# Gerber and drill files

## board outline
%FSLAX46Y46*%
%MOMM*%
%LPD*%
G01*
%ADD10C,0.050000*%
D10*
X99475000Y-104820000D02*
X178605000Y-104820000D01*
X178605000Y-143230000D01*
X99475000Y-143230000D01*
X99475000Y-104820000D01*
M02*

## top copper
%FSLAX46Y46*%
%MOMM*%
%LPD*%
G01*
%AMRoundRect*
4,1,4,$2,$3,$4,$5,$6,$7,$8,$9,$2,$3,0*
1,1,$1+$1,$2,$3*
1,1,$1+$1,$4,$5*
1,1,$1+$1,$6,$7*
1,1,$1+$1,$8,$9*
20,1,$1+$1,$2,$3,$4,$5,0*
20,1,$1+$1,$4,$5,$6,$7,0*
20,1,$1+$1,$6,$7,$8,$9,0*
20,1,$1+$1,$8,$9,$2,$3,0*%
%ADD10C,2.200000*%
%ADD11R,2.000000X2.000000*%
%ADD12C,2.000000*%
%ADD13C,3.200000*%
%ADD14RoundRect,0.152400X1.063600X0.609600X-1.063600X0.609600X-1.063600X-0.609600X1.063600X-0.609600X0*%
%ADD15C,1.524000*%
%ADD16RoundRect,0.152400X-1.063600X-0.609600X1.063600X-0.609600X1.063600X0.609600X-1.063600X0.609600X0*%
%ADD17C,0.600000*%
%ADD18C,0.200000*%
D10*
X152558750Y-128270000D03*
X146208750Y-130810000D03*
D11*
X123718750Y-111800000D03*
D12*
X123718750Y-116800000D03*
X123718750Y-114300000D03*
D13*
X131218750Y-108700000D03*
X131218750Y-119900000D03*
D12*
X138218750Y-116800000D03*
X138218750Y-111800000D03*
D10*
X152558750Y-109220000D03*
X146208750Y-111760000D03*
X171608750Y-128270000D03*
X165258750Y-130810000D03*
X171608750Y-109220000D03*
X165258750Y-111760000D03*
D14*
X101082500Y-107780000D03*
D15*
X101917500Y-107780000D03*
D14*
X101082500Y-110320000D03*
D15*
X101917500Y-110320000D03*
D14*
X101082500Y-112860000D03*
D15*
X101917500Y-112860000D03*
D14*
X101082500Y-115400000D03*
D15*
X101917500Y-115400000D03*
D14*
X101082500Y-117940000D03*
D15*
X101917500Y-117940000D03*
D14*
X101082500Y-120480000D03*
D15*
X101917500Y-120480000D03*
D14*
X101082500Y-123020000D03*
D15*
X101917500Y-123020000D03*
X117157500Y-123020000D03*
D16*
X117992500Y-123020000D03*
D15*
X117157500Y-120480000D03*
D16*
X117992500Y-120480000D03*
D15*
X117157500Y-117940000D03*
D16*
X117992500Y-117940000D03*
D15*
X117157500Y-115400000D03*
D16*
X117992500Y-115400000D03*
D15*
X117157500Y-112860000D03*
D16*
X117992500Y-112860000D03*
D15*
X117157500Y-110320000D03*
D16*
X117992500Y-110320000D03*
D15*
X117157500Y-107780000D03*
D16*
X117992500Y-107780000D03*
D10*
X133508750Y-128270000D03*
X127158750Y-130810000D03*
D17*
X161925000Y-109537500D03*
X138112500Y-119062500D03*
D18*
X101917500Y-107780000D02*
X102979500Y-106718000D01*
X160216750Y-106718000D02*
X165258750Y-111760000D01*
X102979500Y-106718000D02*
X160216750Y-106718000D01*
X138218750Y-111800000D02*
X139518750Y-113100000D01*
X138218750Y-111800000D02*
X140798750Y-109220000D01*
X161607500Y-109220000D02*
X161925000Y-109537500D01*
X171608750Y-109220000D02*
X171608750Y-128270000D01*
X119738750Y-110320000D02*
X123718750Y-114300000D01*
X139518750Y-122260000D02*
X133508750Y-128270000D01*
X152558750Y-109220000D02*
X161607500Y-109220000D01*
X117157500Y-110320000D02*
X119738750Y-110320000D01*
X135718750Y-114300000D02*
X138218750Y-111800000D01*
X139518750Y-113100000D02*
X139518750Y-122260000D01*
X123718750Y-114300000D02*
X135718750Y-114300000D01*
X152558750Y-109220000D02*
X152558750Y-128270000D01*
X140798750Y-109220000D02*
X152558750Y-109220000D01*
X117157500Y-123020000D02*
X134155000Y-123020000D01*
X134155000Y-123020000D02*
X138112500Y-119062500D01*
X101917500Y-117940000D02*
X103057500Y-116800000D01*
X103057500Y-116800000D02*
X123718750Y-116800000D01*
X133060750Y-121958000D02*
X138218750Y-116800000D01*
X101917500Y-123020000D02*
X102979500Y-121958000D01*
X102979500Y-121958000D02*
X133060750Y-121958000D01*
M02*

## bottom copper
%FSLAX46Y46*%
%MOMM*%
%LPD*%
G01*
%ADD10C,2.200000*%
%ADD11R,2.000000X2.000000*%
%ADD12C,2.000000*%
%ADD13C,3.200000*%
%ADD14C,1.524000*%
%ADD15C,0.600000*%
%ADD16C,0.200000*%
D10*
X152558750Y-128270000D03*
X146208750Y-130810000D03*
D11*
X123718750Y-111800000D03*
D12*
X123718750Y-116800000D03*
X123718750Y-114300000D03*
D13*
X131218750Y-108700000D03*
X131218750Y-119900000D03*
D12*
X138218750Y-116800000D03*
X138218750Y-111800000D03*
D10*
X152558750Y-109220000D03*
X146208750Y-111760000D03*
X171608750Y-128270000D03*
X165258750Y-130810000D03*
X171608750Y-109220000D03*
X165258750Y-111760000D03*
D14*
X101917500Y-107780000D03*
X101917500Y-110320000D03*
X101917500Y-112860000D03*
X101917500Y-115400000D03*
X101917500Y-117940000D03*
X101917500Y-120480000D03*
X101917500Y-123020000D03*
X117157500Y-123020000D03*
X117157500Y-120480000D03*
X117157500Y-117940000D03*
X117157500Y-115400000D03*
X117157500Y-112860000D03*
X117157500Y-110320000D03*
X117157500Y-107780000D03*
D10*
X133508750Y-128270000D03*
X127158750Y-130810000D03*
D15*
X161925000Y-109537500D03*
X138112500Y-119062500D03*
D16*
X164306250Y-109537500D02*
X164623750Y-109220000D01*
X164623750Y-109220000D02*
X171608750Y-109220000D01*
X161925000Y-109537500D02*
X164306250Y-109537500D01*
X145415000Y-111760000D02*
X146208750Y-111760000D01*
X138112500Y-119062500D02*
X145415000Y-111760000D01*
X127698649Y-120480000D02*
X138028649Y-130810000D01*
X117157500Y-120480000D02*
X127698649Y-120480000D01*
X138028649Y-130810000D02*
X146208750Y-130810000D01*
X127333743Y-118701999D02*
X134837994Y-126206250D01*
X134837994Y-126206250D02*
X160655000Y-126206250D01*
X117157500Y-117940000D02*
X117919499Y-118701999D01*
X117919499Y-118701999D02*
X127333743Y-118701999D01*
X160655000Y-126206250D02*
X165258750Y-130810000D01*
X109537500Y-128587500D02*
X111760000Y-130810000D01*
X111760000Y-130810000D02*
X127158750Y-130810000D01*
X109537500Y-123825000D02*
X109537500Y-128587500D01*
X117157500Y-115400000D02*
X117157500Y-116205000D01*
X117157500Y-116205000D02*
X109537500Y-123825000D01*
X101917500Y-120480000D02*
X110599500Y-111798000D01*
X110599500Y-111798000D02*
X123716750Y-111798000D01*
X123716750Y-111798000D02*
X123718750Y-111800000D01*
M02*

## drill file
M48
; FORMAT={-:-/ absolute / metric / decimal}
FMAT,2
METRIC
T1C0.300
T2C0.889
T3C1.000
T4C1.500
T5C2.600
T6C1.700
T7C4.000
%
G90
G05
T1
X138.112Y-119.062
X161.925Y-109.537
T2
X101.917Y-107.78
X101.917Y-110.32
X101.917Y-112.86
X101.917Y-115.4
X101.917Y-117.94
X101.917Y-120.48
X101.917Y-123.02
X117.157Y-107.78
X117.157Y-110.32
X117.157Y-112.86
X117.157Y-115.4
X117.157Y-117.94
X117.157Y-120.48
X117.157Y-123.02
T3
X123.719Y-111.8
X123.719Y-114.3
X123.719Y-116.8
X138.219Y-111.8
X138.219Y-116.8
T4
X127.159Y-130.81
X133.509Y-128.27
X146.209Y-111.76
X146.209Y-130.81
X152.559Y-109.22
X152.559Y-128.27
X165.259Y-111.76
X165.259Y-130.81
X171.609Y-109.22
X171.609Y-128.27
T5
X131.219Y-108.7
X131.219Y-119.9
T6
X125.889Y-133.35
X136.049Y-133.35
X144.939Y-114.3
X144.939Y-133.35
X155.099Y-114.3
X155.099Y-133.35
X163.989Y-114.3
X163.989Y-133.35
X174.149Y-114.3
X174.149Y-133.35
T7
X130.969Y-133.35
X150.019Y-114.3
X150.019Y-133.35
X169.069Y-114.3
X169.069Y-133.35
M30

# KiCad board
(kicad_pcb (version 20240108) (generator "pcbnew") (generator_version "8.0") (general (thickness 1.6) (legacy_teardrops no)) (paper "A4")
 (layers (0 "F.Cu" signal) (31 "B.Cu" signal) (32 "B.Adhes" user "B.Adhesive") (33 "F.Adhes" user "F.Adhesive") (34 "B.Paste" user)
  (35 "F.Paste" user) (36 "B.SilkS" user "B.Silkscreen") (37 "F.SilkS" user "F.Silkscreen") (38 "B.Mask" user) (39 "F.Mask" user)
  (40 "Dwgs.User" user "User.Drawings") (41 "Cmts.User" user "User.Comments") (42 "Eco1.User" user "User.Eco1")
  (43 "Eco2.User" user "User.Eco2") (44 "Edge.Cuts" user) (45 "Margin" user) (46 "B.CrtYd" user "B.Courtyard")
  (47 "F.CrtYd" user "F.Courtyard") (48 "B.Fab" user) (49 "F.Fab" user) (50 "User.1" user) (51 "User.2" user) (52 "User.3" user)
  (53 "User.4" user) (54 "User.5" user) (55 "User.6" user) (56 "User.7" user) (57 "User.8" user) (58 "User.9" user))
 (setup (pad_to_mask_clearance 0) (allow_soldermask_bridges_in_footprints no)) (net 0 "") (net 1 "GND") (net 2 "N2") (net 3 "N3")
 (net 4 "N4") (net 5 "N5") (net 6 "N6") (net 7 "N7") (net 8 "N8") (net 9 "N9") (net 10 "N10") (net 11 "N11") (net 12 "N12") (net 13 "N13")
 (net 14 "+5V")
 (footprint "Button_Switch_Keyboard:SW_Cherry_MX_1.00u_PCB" (layer "F.Cu") (at 152.55875 128.27)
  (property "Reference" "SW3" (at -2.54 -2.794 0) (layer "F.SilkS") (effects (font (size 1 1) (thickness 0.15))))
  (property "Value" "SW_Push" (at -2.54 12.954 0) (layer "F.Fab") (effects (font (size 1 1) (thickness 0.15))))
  (pad "" np_thru_hole circle (at -7.62 5.08) (size 1.7 1.7) (drill 1.7) (layers "*.Cu" "*.Mask"))
  (pad "" np_thru_hole circle (at -2.54 5.08) (size 4 4) (drill 4) (layers "*.Cu" "*.Mask"))
  (pad "" np_thru_hole circle (at 2.54 5.08) (size 1.7 1.7) (drill 1.7) (layers "*.Cu" "*.Mask"))
  (pad "1" thru_hole circle (at 0 0) (size 2.2 2.2) (drill 1.5) (layers "*.Cu" "*.Mask") (remove_unused_layers no) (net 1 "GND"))
  (pad "2" thru_hole circle (at -6.35 2.54) (size 2.2 2.2) (drill 1.5) (layers "*.Cu" "*.Mask") (remove_unused_layers no) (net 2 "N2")))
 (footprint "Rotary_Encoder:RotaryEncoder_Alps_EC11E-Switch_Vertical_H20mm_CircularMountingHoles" (layer "F.Cu") (at 123.71875 111.8)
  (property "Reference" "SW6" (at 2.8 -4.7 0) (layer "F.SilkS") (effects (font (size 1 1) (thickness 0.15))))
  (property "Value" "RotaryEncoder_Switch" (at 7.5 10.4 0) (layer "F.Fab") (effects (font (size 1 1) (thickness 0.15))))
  (pad "A" thru_hole rect (at 0 0) (size 2 2) (drill 1) (layers "*.Cu" "*.Mask") (remove_unused_layers no) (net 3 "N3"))
  (pad "B" thru_hole circle (at 0 5) (size 2 2) (drill 1) (layers "*.Cu" "*.Mask") (remove_unused_layers no) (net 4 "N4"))
  (pad "C" thru_hole circle (at 0 2.5) (size 2 2) (drill 1) (layers "*.Cu" "*.Mask") (remove_unused_layers no) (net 1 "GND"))
  (pad "MP" thru_hole circle (at 7.5 -3.1) (size 3.2 3.2) (drill 2.6) (layers "*.Cu" "*.Mask") (remove_unused_layers no))
  (pad "MP" thru_hole circle (at 7.5 8.1) (size 3.2 3.2) (drill 2.6) (layers "*.Cu" "*.Mask") (remove_unused_layers no))
  (pad "S1" thru_hole circle (at 14.5 5) (size 2 2) (drill 1) (layers "*.Cu" "*.Mask") (remove_unused_layers no) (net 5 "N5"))
  (pad "S2" thru_hole circle (at 14.5 0) (size 2 2) (drill 1) (layers "*.Cu" "*.Mask") (remove_unused_layers no) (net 1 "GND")))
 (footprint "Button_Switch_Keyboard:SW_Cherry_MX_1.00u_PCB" (layer "F.Cu") (at 152.55875 109.22)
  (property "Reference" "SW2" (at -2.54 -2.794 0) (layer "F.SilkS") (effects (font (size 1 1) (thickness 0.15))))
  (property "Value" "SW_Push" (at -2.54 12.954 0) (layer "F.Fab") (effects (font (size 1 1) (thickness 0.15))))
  (pad "" np_thru_hole circle (at -7.62 5.08) (size 1.7 1.7) (drill 1.7) (layers "*.Cu" "*.Mask"))
  (pad "" np_thru_hole circle (at -2.54 5.08) (size 4 4) (drill 4) (layers "*.Cu" "*.Mask"))
  (pad "" np_thru_hole circle (at 2.54 5.08) (size 1.7 1.7) (drill 1.7) (layers "*.Cu" "*.Mask"))
  (pad "1" thru_hole circle (at 0 0) (size 2.2 2.2) (drill 1.5) (layers "*.Cu" "*.Mask") (remove_unused_layers no) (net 1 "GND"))
  (pad "2" thru_hole circle (at -6.35 2.54) (size 2.2 2.2) (drill 1.5) (layers "*.Cu" "*.Mask") (remove_unused_layers no) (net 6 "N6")))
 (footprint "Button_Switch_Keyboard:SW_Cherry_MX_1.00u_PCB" (layer "F.Cu") (at 171.60875 128.27)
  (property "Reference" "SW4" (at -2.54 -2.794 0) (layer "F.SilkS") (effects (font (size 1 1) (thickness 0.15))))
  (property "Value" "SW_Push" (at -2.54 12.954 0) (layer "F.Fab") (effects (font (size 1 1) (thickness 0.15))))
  (pad "" np_thru_hole circle (at -7.62 5.08) (size 1.7 1.7) (drill 1.7) (layers "*.Cu" "*.Mask"))
  (pad "" np_thru_hole circle (at -2.54 5.08) (size 4 4) (drill 4) (layers "*.Cu" "*.Mask"))
  (pad "" np_thru_hole circle (at 2.54 5.08) (size 1.7 1.7) (drill 1.7) (layers "*.Cu" "*.Mask"))
  (pad "1" thru_hole circle (at 0 0) (size 2.2 2.2) (drill 1.5) (layers "*.Cu" "*.Mask") (remove_unused_layers no) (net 1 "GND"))
  (pad "2" thru_hole circle (at -6.35 2.54) (size 2.2 2.2) (drill 1.5) (layers "*.Cu" "*.Mask") (remove_unused_layers no) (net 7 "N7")))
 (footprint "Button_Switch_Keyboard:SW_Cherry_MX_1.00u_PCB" (layer "F.Cu") (at 171.60875 109.22)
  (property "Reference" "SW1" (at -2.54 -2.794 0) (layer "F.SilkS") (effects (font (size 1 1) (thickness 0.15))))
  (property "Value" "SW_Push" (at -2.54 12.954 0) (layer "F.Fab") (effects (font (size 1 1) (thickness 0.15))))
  (pad "" np_thru_hole circle (at -7.62 5.08) (size 1.7 1.7) (drill 1.7) (layers "*.Cu" "*.Mask"))
  (pad "" np_thru_hole circle (at -2.54 5.08) (size 4 4) (drill 4) (layers "*.Cu" "*.Mask"))
  (pad "" np_thru_hole circle (at 2.54 5.08) (size 1.7 1.7) (drill 1.7) (layers "*.Cu" "*.Mask"))
  (pad "1" thru_hole circle (at 0 0) (size 2.2 2.2) (drill 1.5) (layers "*.Cu" "*.Mask") (remove_unused_layers no) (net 1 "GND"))
  (pad "2" thru_hole circle (at -6.35 2.54) (size 2.2 2.2) (drill 1.5) (layers "*.Cu" "*.Mask") (remove_unused_layers no) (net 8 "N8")))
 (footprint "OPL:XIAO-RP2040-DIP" (layer "F.Cu") (at 109.5375 115.4)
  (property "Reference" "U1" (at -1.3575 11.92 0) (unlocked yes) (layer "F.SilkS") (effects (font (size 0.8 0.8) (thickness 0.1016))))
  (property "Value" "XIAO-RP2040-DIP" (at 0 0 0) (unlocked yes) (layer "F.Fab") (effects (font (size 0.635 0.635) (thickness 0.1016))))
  (pad "1" smd roundrect (at -8.455 -7.62 180) (size 2.432 1.524) (layers "F.Cu" "F.Mask") (roundrect_rratio 0.1) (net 8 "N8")
   (thermal_bridge_angle 45))
  (pad "1" thru_hole circle (at -7.62 -7.62 180) (size 1.524 1.524) (drill 0.889) (layers "*.Cu" "*.Mask") (remove_unused_layers no)
   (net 8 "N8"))
  (pad "2" smd roundrect (at -8.455 -5.08 180) (size 2.432 1.524) (layers "F.Cu" "F.Mask") (roundrect_rratio 0.1) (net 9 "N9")
   (thermal_bridge_angle 45))
  (pad "2" thru_hole circle (at -7.62 -5.08 180) (size 1.524 1.524) (drill 0.889) (layers "*.Cu" "*.Mask") (remove_unused_layers no)
   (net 9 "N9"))
  (pad "3" smd roundrect (at -8.455 -2.54 180) (size 2.432 1.524) (layers "F.Cu" "F.Mask") (roundrect_rratio 0.1) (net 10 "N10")
   (thermal_bridge_angle 45))
  (pad "3" thru_hole circle (at -7.62 -2.54 180) (size 1.524 1.524) (drill 0.889) (layers "*.Cu" "*.Mask") (remove_unused_layers no)
   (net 10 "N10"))
  (pad "4" smd roundrect (at -8.455 0 180) (size 2.432 1.524) (layers "F.Cu" "F.Mask") (roundrect_rratio 0.1) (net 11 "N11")
   (thermal_bridge_angle 45))
  (pad "4" thru_hole circle (at -7.62 0 180) (size 1.524 1.524) (drill 0.889) (layers "*.Cu" "*.Mask") (remove_unused_layers no)
   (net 11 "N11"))
  (pad "5" smd roundrect (at -8.455 2.54 180) (size 2.432 1.524) (layers "F.Cu" "F.Mask") (roundrect_rratio 0.1) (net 4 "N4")
   (thermal_bridge_angle 45))
  (pad "5" thru_hole circle (at -7.62 2.54 180) (size 1.524 1.524) (drill 0.889) (layers "*.Cu" "*.Mask") (remove_unused_layers no)
   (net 4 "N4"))
  (pad "6" smd roundrect (at -8.455 5.08 180) (size 2.432 1.524) (layers "F.Cu" "F.Mask") (roundrect_rratio 0.1) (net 3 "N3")
   (thermal_bridge_angle 45))
  (pad "6" thru_hole circle (at -7.62 5.08 180) (size 1.524 1.524) (drill 0.889) (layers "*.Cu" "*.Mask") (remove_unused_layers no)
   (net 3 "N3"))
  (pad "7" smd roundrect (at -8.455 7.62 180) (size 2.432 1.524) (layers "F.Cu" "F.Mask") (roundrect_rratio 0.1) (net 5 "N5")
   (thermal_bridge_angle 45))
  (pad "7" thru_hole circle (at -7.62 7.62 180) (size 1.524 1.524) (drill 0.889) (layers "*.Cu" "*.Mask") (remove_unused_layers no)
   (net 5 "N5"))
  (pad "8" thru_hole circle (at 7.62 7.62) (size 1.524 1.524) (drill 0.889) (layers "*.Cu" "*.Mask") (remove_unused_layers no) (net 6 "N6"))
  (pad "8" smd roundrect (at 8.455 7.62) (size 2.432 1.524) (layers "F.Cu" "F.Mask") (roundrect_rratio 0.1) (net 6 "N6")
   (thermal_bridge_angle 45))
  (pad "9" thru_hole circle (at 7.62 5.08) (size 1.524 1.524) (drill 0.889) (layers "*.Cu" "*.Mask") (remove_unused_layers no) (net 2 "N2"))
  (pad "9" smd roundrect (at 8.455 5.08) (size 2.432 1.524) (layers "F.Cu" "F.Mask") (roundrect_rratio 0.1) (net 2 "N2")
   (thermal_bridge_angle 45))
  (pad "10" thru_hole circle (at 7.62 2.54) (size 1.524 1.524) (drill 0.889) (layers "*.Cu" "*.Mask") (remove_unused_layers no) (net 7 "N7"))
  (pad "10" smd roundrect (at 8.455 2.54) (size 2.432 1.524) (layers "F.Cu" "F.Mask") (roundrect_rratio 0.1) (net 7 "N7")
   (thermal_bridge_angle 45))
  (pad "11" thru_hole circle (at 7.62 0) (size 1.524 1.524) (drill 0.889) (layers "*.Cu" "*.Mask") (remove_unused_layers no) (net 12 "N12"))
  (pad "11" smd roundrect (at 8.455 0) (size 2.432 1.524) (layers "F.Cu" "F.Mask") (roundrect_rratio 0.1) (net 12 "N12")
   (thermal_bridge_angle 45))
  (pad "12" thru_hole circle (at 7.62 -2.54) (size 1.524 1.524) (drill 0.889) (layers "*.Cu" "*.Mask") (remove_unused_layers no)
   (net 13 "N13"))
  (pad "12" smd roundrect (at 8.455 -2.54) (size 2.432 1.524) (layers "F.Cu" "F.Mask") (roundrect_rratio 0.1) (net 13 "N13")
   (thermal_bridge_angle 45))
  (pad "13" thru_hole circle (at 7.62 -5.08) (size 1.524 1.524) (drill 0.889) (layers "*.Cu" "*.Mask") (remove_unused_layers no)
   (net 1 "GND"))
  (pad "13" smd roundrect (at 8.455 -5.08) (size 2.432 1.524) (layers "F.Cu" "F.Mask") (roundrect_rratio 0.1) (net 1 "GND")
   (thermal_bridge_angle 45))
  (pad "14" thru_hole circle (at 7.62 -7.62) (size 1.524 1.524) (drill 0.889) (layers "*.Cu" "*.Mask") (remove_unused_layers no)
   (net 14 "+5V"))
  (pad "14" smd roundrect (at 8.455 -7.62) (size 2.432 1.524) (layers "F.Cu" "F.Mask") (roundrect_rratio 0.1) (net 14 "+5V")
   (thermal_bridge_angle 45)))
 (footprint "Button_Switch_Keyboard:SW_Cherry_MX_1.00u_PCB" (layer "F.Cu") (at 133.50875 128.27)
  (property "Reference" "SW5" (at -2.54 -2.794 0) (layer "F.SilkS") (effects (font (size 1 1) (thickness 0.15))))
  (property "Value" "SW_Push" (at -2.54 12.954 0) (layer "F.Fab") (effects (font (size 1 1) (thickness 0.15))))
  (pad "" np_thru_hole circle (at -7.62 5.08) (size 1.7 1.7) (drill 1.7) (layers "*.Cu" "*.Mask"))
  (pad "" np_thru_hole circle (at -2.54 5.08) (size 4 4) (drill 4) (layers "*.Cu" "*.Mask"))
  (pad "" np_thru_hole circle (at 2.54 5.08) (size 1.7 1.7) (drill 1.7) (layers "*.Cu" "*.Mask"))
  (pad "1" thru_hole circle (at 0 0) (size 2.2 2.2) (drill 1.5) (layers "*.Cu" "*.Mask") (remove_unused_layers no) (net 1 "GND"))
  (pad "2" thru_hole circle (at -6.35 2.54) (size 2.2 2.2) (drill 1.5) (layers "*.Cu" "*.Mask") (remove_unused_layers no) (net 12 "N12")))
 (gr_rect (start 99.475 104.82) (end 178.605 143.23) (stroke (width 0.05) (type default)) (fill none) (layer "Edge.Cuts"))
 (segment (start 101.9175 107.78) (end 102.9795 106.718) (width 0.2) (layer "F.Cu") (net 8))
 (segment (start 160.21675 106.718) (end 165.25875 111.76) (width 0.2) (layer "F.Cu") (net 8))
 (segment (start 102.9795 106.718) (end 160.21675 106.718) (width 0.2) (layer "F.Cu") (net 8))
 (segment (start 138.21875 111.8) (end 139.51875 113.1) (width 0.2) (layer "F.Cu") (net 1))
 (segment (start 138.21875 111.8) (end 140.79875 109.22) (width 0.2) (layer "F.Cu") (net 1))
 (segment (start 161.6075 109.22) (end 161.925 109.5375) (width 0.2) (layer "F.Cu") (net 1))
 (segment (start 171.60875 109.22) (end 171.60875 128.27) (width 0.2) (layer "F.Cu") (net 1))
 (segment (start 119.73875 110.32) (end 123.71875 114.3) (width 0.2) (layer "F.Cu") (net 1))
 (segment (start 139.51875 122.26) (end 133.50875 128.27) (width 0.2) (layer "F.Cu") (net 1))
 (segment (start 152.55875 109.22) (end 161.6075 109.22) (width 0.2) (layer "F.Cu") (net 1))
 (segment (start 117.1575 110.32) (end 119.73875 110.32) (width 0.2) (layer "F.Cu") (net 1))
 (segment (start 135.71875 114.3) (end 138.21875 111.8) (width 0.2) (layer "F.Cu") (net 1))
 (segment (start 139.51875 113.1) (end 139.51875 122.26) (width 0.2) (layer "F.Cu") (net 1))
 (segment (start 123.71875 114.3) (end 135.71875 114.3) (width 0.2) (layer "F.Cu") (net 1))
 (segment (start 152.55875 109.22) (end 152.55875 128.27) (width 0.2) (layer "F.Cu") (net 1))
 (segment (start 140.79875 109.22) (end 152.55875 109.22) (width 0.2) (layer "F.Cu") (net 1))
 (via (at 161.925 109.5375) (size 0.6) (drill 0.3) (layers "F.Cu" "B.Cu") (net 1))
 (segment (start 164.30625 109.5375) (end 164.62375 109.22) (width 0.2) (layer "B.Cu") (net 1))
 (segment (start 164.62375 109.22) (end 171.60875 109.22) (width 0.2) (layer "B.Cu") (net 1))
 (segment (start 161.925 109.5375) (end 164.30625 109.5375) (width 0.2) (layer "B.Cu") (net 1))
 (segment (start 117.1575 123.02) (end 134.155 123.02) (width 0.2) (layer "F.Cu") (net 6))
 (segment (start 134.155 123.02) (end 138.1125 119.0625) (width 0.2) (layer "F.Cu") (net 6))
 (via (at 138.1125 119.0625) (size 0.6) (drill 0.3) (layers "F.Cu" "B.Cu") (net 6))
 (segment (start 145.415 111.76) (end 146.20875 111.76) (width 0.2) (layer "B.Cu") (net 6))
 (segment (start 138.1125 119.0625) (end 145.415 111.76) (width 0.2) (layer "B.Cu") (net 6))
 (segment (start 127.698649 120.48) (end 138.028649 130.81) (width 0.2) (layer "B.Cu") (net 2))
 (segment (start 117.1575 120.48) (end 127.698649 120.48) (width 0.2) (layer "B.Cu") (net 2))
 (segment (start 138.028649 130.81) (end 146.20875 130.81) (width 0.2) (layer "B.Cu") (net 2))
 (segment (start 127.333743 118.701999) (end 134.837994 126.20625) (width 0.2) (layer "B.Cu") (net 7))
 (segment (start 134.837994 126.20625) (end 160.655 126.20625) (width 0.2) (layer "B.Cu") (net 7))
 (segment (start 117.1575 117.94) (end 117.919499 118.701999) (width 0.2) (layer "B.Cu") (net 7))
 (segment (start 117.919499 118.701999) (end 127.333743 118.701999) (width 0.2) (layer "B.Cu") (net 7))
 (segment (start 160.655 126.20625) (end 165.25875 130.81) (width 0.2) (layer "B.Cu") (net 7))
 (segment (start 109.5375 128.5875) (end 111.76 130.81) (width 0.2) (layer "B.Cu") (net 12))
 (segment (start 111.76 130.81) (end 127.15875 130.81) (width 0.2) (layer "B.Cu") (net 12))
 (segment (start 109.5375 123.825) (end 109.5375 128.5875) (width 0.2) (layer "B.Cu") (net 12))
 (segment (start 117.1575 115.4) (end 117.1575 116.205) (width 0.2) (layer "B.Cu") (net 12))
 (segment (start 117.1575 116.205) (end 109.5375 123.825) (width 0.2) (layer "B.Cu") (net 12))
 (segment (start 101.9175 117.94) (end 103.0575 116.8) (width 0.2) (layer "F.Cu") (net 4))
 (segment (start 103.0575 116.8) (end 123.71875 116.8) (width 0.2) (layer "F.Cu") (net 4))
 (segment (start 101.9175 120.48) (end 110.5995 111.798) (width 0.2) (layer "B.Cu") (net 3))
 (segment (start 110.5995 111.798) (end 123.71675 111.798) (width 0.2) (layer "B.Cu") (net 3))
 (segment (start 123.71675 111.798) (end 123.71875 111.8) (width 0.2) (layer "B.Cu") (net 3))
 (segment (start 133.06075 121.958) (end 138.21875 116.8) (width 0.2) (layer "F.Cu") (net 5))
 (segment (start 101.9175 123.02) (end 102.9795 121.958) (width 0.2) (layer "F.Cu") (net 5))
 (segment (start 102.9795 121.958) (end 133.06075 121.958) (width 0.2) (layer "F.Cu") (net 5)))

